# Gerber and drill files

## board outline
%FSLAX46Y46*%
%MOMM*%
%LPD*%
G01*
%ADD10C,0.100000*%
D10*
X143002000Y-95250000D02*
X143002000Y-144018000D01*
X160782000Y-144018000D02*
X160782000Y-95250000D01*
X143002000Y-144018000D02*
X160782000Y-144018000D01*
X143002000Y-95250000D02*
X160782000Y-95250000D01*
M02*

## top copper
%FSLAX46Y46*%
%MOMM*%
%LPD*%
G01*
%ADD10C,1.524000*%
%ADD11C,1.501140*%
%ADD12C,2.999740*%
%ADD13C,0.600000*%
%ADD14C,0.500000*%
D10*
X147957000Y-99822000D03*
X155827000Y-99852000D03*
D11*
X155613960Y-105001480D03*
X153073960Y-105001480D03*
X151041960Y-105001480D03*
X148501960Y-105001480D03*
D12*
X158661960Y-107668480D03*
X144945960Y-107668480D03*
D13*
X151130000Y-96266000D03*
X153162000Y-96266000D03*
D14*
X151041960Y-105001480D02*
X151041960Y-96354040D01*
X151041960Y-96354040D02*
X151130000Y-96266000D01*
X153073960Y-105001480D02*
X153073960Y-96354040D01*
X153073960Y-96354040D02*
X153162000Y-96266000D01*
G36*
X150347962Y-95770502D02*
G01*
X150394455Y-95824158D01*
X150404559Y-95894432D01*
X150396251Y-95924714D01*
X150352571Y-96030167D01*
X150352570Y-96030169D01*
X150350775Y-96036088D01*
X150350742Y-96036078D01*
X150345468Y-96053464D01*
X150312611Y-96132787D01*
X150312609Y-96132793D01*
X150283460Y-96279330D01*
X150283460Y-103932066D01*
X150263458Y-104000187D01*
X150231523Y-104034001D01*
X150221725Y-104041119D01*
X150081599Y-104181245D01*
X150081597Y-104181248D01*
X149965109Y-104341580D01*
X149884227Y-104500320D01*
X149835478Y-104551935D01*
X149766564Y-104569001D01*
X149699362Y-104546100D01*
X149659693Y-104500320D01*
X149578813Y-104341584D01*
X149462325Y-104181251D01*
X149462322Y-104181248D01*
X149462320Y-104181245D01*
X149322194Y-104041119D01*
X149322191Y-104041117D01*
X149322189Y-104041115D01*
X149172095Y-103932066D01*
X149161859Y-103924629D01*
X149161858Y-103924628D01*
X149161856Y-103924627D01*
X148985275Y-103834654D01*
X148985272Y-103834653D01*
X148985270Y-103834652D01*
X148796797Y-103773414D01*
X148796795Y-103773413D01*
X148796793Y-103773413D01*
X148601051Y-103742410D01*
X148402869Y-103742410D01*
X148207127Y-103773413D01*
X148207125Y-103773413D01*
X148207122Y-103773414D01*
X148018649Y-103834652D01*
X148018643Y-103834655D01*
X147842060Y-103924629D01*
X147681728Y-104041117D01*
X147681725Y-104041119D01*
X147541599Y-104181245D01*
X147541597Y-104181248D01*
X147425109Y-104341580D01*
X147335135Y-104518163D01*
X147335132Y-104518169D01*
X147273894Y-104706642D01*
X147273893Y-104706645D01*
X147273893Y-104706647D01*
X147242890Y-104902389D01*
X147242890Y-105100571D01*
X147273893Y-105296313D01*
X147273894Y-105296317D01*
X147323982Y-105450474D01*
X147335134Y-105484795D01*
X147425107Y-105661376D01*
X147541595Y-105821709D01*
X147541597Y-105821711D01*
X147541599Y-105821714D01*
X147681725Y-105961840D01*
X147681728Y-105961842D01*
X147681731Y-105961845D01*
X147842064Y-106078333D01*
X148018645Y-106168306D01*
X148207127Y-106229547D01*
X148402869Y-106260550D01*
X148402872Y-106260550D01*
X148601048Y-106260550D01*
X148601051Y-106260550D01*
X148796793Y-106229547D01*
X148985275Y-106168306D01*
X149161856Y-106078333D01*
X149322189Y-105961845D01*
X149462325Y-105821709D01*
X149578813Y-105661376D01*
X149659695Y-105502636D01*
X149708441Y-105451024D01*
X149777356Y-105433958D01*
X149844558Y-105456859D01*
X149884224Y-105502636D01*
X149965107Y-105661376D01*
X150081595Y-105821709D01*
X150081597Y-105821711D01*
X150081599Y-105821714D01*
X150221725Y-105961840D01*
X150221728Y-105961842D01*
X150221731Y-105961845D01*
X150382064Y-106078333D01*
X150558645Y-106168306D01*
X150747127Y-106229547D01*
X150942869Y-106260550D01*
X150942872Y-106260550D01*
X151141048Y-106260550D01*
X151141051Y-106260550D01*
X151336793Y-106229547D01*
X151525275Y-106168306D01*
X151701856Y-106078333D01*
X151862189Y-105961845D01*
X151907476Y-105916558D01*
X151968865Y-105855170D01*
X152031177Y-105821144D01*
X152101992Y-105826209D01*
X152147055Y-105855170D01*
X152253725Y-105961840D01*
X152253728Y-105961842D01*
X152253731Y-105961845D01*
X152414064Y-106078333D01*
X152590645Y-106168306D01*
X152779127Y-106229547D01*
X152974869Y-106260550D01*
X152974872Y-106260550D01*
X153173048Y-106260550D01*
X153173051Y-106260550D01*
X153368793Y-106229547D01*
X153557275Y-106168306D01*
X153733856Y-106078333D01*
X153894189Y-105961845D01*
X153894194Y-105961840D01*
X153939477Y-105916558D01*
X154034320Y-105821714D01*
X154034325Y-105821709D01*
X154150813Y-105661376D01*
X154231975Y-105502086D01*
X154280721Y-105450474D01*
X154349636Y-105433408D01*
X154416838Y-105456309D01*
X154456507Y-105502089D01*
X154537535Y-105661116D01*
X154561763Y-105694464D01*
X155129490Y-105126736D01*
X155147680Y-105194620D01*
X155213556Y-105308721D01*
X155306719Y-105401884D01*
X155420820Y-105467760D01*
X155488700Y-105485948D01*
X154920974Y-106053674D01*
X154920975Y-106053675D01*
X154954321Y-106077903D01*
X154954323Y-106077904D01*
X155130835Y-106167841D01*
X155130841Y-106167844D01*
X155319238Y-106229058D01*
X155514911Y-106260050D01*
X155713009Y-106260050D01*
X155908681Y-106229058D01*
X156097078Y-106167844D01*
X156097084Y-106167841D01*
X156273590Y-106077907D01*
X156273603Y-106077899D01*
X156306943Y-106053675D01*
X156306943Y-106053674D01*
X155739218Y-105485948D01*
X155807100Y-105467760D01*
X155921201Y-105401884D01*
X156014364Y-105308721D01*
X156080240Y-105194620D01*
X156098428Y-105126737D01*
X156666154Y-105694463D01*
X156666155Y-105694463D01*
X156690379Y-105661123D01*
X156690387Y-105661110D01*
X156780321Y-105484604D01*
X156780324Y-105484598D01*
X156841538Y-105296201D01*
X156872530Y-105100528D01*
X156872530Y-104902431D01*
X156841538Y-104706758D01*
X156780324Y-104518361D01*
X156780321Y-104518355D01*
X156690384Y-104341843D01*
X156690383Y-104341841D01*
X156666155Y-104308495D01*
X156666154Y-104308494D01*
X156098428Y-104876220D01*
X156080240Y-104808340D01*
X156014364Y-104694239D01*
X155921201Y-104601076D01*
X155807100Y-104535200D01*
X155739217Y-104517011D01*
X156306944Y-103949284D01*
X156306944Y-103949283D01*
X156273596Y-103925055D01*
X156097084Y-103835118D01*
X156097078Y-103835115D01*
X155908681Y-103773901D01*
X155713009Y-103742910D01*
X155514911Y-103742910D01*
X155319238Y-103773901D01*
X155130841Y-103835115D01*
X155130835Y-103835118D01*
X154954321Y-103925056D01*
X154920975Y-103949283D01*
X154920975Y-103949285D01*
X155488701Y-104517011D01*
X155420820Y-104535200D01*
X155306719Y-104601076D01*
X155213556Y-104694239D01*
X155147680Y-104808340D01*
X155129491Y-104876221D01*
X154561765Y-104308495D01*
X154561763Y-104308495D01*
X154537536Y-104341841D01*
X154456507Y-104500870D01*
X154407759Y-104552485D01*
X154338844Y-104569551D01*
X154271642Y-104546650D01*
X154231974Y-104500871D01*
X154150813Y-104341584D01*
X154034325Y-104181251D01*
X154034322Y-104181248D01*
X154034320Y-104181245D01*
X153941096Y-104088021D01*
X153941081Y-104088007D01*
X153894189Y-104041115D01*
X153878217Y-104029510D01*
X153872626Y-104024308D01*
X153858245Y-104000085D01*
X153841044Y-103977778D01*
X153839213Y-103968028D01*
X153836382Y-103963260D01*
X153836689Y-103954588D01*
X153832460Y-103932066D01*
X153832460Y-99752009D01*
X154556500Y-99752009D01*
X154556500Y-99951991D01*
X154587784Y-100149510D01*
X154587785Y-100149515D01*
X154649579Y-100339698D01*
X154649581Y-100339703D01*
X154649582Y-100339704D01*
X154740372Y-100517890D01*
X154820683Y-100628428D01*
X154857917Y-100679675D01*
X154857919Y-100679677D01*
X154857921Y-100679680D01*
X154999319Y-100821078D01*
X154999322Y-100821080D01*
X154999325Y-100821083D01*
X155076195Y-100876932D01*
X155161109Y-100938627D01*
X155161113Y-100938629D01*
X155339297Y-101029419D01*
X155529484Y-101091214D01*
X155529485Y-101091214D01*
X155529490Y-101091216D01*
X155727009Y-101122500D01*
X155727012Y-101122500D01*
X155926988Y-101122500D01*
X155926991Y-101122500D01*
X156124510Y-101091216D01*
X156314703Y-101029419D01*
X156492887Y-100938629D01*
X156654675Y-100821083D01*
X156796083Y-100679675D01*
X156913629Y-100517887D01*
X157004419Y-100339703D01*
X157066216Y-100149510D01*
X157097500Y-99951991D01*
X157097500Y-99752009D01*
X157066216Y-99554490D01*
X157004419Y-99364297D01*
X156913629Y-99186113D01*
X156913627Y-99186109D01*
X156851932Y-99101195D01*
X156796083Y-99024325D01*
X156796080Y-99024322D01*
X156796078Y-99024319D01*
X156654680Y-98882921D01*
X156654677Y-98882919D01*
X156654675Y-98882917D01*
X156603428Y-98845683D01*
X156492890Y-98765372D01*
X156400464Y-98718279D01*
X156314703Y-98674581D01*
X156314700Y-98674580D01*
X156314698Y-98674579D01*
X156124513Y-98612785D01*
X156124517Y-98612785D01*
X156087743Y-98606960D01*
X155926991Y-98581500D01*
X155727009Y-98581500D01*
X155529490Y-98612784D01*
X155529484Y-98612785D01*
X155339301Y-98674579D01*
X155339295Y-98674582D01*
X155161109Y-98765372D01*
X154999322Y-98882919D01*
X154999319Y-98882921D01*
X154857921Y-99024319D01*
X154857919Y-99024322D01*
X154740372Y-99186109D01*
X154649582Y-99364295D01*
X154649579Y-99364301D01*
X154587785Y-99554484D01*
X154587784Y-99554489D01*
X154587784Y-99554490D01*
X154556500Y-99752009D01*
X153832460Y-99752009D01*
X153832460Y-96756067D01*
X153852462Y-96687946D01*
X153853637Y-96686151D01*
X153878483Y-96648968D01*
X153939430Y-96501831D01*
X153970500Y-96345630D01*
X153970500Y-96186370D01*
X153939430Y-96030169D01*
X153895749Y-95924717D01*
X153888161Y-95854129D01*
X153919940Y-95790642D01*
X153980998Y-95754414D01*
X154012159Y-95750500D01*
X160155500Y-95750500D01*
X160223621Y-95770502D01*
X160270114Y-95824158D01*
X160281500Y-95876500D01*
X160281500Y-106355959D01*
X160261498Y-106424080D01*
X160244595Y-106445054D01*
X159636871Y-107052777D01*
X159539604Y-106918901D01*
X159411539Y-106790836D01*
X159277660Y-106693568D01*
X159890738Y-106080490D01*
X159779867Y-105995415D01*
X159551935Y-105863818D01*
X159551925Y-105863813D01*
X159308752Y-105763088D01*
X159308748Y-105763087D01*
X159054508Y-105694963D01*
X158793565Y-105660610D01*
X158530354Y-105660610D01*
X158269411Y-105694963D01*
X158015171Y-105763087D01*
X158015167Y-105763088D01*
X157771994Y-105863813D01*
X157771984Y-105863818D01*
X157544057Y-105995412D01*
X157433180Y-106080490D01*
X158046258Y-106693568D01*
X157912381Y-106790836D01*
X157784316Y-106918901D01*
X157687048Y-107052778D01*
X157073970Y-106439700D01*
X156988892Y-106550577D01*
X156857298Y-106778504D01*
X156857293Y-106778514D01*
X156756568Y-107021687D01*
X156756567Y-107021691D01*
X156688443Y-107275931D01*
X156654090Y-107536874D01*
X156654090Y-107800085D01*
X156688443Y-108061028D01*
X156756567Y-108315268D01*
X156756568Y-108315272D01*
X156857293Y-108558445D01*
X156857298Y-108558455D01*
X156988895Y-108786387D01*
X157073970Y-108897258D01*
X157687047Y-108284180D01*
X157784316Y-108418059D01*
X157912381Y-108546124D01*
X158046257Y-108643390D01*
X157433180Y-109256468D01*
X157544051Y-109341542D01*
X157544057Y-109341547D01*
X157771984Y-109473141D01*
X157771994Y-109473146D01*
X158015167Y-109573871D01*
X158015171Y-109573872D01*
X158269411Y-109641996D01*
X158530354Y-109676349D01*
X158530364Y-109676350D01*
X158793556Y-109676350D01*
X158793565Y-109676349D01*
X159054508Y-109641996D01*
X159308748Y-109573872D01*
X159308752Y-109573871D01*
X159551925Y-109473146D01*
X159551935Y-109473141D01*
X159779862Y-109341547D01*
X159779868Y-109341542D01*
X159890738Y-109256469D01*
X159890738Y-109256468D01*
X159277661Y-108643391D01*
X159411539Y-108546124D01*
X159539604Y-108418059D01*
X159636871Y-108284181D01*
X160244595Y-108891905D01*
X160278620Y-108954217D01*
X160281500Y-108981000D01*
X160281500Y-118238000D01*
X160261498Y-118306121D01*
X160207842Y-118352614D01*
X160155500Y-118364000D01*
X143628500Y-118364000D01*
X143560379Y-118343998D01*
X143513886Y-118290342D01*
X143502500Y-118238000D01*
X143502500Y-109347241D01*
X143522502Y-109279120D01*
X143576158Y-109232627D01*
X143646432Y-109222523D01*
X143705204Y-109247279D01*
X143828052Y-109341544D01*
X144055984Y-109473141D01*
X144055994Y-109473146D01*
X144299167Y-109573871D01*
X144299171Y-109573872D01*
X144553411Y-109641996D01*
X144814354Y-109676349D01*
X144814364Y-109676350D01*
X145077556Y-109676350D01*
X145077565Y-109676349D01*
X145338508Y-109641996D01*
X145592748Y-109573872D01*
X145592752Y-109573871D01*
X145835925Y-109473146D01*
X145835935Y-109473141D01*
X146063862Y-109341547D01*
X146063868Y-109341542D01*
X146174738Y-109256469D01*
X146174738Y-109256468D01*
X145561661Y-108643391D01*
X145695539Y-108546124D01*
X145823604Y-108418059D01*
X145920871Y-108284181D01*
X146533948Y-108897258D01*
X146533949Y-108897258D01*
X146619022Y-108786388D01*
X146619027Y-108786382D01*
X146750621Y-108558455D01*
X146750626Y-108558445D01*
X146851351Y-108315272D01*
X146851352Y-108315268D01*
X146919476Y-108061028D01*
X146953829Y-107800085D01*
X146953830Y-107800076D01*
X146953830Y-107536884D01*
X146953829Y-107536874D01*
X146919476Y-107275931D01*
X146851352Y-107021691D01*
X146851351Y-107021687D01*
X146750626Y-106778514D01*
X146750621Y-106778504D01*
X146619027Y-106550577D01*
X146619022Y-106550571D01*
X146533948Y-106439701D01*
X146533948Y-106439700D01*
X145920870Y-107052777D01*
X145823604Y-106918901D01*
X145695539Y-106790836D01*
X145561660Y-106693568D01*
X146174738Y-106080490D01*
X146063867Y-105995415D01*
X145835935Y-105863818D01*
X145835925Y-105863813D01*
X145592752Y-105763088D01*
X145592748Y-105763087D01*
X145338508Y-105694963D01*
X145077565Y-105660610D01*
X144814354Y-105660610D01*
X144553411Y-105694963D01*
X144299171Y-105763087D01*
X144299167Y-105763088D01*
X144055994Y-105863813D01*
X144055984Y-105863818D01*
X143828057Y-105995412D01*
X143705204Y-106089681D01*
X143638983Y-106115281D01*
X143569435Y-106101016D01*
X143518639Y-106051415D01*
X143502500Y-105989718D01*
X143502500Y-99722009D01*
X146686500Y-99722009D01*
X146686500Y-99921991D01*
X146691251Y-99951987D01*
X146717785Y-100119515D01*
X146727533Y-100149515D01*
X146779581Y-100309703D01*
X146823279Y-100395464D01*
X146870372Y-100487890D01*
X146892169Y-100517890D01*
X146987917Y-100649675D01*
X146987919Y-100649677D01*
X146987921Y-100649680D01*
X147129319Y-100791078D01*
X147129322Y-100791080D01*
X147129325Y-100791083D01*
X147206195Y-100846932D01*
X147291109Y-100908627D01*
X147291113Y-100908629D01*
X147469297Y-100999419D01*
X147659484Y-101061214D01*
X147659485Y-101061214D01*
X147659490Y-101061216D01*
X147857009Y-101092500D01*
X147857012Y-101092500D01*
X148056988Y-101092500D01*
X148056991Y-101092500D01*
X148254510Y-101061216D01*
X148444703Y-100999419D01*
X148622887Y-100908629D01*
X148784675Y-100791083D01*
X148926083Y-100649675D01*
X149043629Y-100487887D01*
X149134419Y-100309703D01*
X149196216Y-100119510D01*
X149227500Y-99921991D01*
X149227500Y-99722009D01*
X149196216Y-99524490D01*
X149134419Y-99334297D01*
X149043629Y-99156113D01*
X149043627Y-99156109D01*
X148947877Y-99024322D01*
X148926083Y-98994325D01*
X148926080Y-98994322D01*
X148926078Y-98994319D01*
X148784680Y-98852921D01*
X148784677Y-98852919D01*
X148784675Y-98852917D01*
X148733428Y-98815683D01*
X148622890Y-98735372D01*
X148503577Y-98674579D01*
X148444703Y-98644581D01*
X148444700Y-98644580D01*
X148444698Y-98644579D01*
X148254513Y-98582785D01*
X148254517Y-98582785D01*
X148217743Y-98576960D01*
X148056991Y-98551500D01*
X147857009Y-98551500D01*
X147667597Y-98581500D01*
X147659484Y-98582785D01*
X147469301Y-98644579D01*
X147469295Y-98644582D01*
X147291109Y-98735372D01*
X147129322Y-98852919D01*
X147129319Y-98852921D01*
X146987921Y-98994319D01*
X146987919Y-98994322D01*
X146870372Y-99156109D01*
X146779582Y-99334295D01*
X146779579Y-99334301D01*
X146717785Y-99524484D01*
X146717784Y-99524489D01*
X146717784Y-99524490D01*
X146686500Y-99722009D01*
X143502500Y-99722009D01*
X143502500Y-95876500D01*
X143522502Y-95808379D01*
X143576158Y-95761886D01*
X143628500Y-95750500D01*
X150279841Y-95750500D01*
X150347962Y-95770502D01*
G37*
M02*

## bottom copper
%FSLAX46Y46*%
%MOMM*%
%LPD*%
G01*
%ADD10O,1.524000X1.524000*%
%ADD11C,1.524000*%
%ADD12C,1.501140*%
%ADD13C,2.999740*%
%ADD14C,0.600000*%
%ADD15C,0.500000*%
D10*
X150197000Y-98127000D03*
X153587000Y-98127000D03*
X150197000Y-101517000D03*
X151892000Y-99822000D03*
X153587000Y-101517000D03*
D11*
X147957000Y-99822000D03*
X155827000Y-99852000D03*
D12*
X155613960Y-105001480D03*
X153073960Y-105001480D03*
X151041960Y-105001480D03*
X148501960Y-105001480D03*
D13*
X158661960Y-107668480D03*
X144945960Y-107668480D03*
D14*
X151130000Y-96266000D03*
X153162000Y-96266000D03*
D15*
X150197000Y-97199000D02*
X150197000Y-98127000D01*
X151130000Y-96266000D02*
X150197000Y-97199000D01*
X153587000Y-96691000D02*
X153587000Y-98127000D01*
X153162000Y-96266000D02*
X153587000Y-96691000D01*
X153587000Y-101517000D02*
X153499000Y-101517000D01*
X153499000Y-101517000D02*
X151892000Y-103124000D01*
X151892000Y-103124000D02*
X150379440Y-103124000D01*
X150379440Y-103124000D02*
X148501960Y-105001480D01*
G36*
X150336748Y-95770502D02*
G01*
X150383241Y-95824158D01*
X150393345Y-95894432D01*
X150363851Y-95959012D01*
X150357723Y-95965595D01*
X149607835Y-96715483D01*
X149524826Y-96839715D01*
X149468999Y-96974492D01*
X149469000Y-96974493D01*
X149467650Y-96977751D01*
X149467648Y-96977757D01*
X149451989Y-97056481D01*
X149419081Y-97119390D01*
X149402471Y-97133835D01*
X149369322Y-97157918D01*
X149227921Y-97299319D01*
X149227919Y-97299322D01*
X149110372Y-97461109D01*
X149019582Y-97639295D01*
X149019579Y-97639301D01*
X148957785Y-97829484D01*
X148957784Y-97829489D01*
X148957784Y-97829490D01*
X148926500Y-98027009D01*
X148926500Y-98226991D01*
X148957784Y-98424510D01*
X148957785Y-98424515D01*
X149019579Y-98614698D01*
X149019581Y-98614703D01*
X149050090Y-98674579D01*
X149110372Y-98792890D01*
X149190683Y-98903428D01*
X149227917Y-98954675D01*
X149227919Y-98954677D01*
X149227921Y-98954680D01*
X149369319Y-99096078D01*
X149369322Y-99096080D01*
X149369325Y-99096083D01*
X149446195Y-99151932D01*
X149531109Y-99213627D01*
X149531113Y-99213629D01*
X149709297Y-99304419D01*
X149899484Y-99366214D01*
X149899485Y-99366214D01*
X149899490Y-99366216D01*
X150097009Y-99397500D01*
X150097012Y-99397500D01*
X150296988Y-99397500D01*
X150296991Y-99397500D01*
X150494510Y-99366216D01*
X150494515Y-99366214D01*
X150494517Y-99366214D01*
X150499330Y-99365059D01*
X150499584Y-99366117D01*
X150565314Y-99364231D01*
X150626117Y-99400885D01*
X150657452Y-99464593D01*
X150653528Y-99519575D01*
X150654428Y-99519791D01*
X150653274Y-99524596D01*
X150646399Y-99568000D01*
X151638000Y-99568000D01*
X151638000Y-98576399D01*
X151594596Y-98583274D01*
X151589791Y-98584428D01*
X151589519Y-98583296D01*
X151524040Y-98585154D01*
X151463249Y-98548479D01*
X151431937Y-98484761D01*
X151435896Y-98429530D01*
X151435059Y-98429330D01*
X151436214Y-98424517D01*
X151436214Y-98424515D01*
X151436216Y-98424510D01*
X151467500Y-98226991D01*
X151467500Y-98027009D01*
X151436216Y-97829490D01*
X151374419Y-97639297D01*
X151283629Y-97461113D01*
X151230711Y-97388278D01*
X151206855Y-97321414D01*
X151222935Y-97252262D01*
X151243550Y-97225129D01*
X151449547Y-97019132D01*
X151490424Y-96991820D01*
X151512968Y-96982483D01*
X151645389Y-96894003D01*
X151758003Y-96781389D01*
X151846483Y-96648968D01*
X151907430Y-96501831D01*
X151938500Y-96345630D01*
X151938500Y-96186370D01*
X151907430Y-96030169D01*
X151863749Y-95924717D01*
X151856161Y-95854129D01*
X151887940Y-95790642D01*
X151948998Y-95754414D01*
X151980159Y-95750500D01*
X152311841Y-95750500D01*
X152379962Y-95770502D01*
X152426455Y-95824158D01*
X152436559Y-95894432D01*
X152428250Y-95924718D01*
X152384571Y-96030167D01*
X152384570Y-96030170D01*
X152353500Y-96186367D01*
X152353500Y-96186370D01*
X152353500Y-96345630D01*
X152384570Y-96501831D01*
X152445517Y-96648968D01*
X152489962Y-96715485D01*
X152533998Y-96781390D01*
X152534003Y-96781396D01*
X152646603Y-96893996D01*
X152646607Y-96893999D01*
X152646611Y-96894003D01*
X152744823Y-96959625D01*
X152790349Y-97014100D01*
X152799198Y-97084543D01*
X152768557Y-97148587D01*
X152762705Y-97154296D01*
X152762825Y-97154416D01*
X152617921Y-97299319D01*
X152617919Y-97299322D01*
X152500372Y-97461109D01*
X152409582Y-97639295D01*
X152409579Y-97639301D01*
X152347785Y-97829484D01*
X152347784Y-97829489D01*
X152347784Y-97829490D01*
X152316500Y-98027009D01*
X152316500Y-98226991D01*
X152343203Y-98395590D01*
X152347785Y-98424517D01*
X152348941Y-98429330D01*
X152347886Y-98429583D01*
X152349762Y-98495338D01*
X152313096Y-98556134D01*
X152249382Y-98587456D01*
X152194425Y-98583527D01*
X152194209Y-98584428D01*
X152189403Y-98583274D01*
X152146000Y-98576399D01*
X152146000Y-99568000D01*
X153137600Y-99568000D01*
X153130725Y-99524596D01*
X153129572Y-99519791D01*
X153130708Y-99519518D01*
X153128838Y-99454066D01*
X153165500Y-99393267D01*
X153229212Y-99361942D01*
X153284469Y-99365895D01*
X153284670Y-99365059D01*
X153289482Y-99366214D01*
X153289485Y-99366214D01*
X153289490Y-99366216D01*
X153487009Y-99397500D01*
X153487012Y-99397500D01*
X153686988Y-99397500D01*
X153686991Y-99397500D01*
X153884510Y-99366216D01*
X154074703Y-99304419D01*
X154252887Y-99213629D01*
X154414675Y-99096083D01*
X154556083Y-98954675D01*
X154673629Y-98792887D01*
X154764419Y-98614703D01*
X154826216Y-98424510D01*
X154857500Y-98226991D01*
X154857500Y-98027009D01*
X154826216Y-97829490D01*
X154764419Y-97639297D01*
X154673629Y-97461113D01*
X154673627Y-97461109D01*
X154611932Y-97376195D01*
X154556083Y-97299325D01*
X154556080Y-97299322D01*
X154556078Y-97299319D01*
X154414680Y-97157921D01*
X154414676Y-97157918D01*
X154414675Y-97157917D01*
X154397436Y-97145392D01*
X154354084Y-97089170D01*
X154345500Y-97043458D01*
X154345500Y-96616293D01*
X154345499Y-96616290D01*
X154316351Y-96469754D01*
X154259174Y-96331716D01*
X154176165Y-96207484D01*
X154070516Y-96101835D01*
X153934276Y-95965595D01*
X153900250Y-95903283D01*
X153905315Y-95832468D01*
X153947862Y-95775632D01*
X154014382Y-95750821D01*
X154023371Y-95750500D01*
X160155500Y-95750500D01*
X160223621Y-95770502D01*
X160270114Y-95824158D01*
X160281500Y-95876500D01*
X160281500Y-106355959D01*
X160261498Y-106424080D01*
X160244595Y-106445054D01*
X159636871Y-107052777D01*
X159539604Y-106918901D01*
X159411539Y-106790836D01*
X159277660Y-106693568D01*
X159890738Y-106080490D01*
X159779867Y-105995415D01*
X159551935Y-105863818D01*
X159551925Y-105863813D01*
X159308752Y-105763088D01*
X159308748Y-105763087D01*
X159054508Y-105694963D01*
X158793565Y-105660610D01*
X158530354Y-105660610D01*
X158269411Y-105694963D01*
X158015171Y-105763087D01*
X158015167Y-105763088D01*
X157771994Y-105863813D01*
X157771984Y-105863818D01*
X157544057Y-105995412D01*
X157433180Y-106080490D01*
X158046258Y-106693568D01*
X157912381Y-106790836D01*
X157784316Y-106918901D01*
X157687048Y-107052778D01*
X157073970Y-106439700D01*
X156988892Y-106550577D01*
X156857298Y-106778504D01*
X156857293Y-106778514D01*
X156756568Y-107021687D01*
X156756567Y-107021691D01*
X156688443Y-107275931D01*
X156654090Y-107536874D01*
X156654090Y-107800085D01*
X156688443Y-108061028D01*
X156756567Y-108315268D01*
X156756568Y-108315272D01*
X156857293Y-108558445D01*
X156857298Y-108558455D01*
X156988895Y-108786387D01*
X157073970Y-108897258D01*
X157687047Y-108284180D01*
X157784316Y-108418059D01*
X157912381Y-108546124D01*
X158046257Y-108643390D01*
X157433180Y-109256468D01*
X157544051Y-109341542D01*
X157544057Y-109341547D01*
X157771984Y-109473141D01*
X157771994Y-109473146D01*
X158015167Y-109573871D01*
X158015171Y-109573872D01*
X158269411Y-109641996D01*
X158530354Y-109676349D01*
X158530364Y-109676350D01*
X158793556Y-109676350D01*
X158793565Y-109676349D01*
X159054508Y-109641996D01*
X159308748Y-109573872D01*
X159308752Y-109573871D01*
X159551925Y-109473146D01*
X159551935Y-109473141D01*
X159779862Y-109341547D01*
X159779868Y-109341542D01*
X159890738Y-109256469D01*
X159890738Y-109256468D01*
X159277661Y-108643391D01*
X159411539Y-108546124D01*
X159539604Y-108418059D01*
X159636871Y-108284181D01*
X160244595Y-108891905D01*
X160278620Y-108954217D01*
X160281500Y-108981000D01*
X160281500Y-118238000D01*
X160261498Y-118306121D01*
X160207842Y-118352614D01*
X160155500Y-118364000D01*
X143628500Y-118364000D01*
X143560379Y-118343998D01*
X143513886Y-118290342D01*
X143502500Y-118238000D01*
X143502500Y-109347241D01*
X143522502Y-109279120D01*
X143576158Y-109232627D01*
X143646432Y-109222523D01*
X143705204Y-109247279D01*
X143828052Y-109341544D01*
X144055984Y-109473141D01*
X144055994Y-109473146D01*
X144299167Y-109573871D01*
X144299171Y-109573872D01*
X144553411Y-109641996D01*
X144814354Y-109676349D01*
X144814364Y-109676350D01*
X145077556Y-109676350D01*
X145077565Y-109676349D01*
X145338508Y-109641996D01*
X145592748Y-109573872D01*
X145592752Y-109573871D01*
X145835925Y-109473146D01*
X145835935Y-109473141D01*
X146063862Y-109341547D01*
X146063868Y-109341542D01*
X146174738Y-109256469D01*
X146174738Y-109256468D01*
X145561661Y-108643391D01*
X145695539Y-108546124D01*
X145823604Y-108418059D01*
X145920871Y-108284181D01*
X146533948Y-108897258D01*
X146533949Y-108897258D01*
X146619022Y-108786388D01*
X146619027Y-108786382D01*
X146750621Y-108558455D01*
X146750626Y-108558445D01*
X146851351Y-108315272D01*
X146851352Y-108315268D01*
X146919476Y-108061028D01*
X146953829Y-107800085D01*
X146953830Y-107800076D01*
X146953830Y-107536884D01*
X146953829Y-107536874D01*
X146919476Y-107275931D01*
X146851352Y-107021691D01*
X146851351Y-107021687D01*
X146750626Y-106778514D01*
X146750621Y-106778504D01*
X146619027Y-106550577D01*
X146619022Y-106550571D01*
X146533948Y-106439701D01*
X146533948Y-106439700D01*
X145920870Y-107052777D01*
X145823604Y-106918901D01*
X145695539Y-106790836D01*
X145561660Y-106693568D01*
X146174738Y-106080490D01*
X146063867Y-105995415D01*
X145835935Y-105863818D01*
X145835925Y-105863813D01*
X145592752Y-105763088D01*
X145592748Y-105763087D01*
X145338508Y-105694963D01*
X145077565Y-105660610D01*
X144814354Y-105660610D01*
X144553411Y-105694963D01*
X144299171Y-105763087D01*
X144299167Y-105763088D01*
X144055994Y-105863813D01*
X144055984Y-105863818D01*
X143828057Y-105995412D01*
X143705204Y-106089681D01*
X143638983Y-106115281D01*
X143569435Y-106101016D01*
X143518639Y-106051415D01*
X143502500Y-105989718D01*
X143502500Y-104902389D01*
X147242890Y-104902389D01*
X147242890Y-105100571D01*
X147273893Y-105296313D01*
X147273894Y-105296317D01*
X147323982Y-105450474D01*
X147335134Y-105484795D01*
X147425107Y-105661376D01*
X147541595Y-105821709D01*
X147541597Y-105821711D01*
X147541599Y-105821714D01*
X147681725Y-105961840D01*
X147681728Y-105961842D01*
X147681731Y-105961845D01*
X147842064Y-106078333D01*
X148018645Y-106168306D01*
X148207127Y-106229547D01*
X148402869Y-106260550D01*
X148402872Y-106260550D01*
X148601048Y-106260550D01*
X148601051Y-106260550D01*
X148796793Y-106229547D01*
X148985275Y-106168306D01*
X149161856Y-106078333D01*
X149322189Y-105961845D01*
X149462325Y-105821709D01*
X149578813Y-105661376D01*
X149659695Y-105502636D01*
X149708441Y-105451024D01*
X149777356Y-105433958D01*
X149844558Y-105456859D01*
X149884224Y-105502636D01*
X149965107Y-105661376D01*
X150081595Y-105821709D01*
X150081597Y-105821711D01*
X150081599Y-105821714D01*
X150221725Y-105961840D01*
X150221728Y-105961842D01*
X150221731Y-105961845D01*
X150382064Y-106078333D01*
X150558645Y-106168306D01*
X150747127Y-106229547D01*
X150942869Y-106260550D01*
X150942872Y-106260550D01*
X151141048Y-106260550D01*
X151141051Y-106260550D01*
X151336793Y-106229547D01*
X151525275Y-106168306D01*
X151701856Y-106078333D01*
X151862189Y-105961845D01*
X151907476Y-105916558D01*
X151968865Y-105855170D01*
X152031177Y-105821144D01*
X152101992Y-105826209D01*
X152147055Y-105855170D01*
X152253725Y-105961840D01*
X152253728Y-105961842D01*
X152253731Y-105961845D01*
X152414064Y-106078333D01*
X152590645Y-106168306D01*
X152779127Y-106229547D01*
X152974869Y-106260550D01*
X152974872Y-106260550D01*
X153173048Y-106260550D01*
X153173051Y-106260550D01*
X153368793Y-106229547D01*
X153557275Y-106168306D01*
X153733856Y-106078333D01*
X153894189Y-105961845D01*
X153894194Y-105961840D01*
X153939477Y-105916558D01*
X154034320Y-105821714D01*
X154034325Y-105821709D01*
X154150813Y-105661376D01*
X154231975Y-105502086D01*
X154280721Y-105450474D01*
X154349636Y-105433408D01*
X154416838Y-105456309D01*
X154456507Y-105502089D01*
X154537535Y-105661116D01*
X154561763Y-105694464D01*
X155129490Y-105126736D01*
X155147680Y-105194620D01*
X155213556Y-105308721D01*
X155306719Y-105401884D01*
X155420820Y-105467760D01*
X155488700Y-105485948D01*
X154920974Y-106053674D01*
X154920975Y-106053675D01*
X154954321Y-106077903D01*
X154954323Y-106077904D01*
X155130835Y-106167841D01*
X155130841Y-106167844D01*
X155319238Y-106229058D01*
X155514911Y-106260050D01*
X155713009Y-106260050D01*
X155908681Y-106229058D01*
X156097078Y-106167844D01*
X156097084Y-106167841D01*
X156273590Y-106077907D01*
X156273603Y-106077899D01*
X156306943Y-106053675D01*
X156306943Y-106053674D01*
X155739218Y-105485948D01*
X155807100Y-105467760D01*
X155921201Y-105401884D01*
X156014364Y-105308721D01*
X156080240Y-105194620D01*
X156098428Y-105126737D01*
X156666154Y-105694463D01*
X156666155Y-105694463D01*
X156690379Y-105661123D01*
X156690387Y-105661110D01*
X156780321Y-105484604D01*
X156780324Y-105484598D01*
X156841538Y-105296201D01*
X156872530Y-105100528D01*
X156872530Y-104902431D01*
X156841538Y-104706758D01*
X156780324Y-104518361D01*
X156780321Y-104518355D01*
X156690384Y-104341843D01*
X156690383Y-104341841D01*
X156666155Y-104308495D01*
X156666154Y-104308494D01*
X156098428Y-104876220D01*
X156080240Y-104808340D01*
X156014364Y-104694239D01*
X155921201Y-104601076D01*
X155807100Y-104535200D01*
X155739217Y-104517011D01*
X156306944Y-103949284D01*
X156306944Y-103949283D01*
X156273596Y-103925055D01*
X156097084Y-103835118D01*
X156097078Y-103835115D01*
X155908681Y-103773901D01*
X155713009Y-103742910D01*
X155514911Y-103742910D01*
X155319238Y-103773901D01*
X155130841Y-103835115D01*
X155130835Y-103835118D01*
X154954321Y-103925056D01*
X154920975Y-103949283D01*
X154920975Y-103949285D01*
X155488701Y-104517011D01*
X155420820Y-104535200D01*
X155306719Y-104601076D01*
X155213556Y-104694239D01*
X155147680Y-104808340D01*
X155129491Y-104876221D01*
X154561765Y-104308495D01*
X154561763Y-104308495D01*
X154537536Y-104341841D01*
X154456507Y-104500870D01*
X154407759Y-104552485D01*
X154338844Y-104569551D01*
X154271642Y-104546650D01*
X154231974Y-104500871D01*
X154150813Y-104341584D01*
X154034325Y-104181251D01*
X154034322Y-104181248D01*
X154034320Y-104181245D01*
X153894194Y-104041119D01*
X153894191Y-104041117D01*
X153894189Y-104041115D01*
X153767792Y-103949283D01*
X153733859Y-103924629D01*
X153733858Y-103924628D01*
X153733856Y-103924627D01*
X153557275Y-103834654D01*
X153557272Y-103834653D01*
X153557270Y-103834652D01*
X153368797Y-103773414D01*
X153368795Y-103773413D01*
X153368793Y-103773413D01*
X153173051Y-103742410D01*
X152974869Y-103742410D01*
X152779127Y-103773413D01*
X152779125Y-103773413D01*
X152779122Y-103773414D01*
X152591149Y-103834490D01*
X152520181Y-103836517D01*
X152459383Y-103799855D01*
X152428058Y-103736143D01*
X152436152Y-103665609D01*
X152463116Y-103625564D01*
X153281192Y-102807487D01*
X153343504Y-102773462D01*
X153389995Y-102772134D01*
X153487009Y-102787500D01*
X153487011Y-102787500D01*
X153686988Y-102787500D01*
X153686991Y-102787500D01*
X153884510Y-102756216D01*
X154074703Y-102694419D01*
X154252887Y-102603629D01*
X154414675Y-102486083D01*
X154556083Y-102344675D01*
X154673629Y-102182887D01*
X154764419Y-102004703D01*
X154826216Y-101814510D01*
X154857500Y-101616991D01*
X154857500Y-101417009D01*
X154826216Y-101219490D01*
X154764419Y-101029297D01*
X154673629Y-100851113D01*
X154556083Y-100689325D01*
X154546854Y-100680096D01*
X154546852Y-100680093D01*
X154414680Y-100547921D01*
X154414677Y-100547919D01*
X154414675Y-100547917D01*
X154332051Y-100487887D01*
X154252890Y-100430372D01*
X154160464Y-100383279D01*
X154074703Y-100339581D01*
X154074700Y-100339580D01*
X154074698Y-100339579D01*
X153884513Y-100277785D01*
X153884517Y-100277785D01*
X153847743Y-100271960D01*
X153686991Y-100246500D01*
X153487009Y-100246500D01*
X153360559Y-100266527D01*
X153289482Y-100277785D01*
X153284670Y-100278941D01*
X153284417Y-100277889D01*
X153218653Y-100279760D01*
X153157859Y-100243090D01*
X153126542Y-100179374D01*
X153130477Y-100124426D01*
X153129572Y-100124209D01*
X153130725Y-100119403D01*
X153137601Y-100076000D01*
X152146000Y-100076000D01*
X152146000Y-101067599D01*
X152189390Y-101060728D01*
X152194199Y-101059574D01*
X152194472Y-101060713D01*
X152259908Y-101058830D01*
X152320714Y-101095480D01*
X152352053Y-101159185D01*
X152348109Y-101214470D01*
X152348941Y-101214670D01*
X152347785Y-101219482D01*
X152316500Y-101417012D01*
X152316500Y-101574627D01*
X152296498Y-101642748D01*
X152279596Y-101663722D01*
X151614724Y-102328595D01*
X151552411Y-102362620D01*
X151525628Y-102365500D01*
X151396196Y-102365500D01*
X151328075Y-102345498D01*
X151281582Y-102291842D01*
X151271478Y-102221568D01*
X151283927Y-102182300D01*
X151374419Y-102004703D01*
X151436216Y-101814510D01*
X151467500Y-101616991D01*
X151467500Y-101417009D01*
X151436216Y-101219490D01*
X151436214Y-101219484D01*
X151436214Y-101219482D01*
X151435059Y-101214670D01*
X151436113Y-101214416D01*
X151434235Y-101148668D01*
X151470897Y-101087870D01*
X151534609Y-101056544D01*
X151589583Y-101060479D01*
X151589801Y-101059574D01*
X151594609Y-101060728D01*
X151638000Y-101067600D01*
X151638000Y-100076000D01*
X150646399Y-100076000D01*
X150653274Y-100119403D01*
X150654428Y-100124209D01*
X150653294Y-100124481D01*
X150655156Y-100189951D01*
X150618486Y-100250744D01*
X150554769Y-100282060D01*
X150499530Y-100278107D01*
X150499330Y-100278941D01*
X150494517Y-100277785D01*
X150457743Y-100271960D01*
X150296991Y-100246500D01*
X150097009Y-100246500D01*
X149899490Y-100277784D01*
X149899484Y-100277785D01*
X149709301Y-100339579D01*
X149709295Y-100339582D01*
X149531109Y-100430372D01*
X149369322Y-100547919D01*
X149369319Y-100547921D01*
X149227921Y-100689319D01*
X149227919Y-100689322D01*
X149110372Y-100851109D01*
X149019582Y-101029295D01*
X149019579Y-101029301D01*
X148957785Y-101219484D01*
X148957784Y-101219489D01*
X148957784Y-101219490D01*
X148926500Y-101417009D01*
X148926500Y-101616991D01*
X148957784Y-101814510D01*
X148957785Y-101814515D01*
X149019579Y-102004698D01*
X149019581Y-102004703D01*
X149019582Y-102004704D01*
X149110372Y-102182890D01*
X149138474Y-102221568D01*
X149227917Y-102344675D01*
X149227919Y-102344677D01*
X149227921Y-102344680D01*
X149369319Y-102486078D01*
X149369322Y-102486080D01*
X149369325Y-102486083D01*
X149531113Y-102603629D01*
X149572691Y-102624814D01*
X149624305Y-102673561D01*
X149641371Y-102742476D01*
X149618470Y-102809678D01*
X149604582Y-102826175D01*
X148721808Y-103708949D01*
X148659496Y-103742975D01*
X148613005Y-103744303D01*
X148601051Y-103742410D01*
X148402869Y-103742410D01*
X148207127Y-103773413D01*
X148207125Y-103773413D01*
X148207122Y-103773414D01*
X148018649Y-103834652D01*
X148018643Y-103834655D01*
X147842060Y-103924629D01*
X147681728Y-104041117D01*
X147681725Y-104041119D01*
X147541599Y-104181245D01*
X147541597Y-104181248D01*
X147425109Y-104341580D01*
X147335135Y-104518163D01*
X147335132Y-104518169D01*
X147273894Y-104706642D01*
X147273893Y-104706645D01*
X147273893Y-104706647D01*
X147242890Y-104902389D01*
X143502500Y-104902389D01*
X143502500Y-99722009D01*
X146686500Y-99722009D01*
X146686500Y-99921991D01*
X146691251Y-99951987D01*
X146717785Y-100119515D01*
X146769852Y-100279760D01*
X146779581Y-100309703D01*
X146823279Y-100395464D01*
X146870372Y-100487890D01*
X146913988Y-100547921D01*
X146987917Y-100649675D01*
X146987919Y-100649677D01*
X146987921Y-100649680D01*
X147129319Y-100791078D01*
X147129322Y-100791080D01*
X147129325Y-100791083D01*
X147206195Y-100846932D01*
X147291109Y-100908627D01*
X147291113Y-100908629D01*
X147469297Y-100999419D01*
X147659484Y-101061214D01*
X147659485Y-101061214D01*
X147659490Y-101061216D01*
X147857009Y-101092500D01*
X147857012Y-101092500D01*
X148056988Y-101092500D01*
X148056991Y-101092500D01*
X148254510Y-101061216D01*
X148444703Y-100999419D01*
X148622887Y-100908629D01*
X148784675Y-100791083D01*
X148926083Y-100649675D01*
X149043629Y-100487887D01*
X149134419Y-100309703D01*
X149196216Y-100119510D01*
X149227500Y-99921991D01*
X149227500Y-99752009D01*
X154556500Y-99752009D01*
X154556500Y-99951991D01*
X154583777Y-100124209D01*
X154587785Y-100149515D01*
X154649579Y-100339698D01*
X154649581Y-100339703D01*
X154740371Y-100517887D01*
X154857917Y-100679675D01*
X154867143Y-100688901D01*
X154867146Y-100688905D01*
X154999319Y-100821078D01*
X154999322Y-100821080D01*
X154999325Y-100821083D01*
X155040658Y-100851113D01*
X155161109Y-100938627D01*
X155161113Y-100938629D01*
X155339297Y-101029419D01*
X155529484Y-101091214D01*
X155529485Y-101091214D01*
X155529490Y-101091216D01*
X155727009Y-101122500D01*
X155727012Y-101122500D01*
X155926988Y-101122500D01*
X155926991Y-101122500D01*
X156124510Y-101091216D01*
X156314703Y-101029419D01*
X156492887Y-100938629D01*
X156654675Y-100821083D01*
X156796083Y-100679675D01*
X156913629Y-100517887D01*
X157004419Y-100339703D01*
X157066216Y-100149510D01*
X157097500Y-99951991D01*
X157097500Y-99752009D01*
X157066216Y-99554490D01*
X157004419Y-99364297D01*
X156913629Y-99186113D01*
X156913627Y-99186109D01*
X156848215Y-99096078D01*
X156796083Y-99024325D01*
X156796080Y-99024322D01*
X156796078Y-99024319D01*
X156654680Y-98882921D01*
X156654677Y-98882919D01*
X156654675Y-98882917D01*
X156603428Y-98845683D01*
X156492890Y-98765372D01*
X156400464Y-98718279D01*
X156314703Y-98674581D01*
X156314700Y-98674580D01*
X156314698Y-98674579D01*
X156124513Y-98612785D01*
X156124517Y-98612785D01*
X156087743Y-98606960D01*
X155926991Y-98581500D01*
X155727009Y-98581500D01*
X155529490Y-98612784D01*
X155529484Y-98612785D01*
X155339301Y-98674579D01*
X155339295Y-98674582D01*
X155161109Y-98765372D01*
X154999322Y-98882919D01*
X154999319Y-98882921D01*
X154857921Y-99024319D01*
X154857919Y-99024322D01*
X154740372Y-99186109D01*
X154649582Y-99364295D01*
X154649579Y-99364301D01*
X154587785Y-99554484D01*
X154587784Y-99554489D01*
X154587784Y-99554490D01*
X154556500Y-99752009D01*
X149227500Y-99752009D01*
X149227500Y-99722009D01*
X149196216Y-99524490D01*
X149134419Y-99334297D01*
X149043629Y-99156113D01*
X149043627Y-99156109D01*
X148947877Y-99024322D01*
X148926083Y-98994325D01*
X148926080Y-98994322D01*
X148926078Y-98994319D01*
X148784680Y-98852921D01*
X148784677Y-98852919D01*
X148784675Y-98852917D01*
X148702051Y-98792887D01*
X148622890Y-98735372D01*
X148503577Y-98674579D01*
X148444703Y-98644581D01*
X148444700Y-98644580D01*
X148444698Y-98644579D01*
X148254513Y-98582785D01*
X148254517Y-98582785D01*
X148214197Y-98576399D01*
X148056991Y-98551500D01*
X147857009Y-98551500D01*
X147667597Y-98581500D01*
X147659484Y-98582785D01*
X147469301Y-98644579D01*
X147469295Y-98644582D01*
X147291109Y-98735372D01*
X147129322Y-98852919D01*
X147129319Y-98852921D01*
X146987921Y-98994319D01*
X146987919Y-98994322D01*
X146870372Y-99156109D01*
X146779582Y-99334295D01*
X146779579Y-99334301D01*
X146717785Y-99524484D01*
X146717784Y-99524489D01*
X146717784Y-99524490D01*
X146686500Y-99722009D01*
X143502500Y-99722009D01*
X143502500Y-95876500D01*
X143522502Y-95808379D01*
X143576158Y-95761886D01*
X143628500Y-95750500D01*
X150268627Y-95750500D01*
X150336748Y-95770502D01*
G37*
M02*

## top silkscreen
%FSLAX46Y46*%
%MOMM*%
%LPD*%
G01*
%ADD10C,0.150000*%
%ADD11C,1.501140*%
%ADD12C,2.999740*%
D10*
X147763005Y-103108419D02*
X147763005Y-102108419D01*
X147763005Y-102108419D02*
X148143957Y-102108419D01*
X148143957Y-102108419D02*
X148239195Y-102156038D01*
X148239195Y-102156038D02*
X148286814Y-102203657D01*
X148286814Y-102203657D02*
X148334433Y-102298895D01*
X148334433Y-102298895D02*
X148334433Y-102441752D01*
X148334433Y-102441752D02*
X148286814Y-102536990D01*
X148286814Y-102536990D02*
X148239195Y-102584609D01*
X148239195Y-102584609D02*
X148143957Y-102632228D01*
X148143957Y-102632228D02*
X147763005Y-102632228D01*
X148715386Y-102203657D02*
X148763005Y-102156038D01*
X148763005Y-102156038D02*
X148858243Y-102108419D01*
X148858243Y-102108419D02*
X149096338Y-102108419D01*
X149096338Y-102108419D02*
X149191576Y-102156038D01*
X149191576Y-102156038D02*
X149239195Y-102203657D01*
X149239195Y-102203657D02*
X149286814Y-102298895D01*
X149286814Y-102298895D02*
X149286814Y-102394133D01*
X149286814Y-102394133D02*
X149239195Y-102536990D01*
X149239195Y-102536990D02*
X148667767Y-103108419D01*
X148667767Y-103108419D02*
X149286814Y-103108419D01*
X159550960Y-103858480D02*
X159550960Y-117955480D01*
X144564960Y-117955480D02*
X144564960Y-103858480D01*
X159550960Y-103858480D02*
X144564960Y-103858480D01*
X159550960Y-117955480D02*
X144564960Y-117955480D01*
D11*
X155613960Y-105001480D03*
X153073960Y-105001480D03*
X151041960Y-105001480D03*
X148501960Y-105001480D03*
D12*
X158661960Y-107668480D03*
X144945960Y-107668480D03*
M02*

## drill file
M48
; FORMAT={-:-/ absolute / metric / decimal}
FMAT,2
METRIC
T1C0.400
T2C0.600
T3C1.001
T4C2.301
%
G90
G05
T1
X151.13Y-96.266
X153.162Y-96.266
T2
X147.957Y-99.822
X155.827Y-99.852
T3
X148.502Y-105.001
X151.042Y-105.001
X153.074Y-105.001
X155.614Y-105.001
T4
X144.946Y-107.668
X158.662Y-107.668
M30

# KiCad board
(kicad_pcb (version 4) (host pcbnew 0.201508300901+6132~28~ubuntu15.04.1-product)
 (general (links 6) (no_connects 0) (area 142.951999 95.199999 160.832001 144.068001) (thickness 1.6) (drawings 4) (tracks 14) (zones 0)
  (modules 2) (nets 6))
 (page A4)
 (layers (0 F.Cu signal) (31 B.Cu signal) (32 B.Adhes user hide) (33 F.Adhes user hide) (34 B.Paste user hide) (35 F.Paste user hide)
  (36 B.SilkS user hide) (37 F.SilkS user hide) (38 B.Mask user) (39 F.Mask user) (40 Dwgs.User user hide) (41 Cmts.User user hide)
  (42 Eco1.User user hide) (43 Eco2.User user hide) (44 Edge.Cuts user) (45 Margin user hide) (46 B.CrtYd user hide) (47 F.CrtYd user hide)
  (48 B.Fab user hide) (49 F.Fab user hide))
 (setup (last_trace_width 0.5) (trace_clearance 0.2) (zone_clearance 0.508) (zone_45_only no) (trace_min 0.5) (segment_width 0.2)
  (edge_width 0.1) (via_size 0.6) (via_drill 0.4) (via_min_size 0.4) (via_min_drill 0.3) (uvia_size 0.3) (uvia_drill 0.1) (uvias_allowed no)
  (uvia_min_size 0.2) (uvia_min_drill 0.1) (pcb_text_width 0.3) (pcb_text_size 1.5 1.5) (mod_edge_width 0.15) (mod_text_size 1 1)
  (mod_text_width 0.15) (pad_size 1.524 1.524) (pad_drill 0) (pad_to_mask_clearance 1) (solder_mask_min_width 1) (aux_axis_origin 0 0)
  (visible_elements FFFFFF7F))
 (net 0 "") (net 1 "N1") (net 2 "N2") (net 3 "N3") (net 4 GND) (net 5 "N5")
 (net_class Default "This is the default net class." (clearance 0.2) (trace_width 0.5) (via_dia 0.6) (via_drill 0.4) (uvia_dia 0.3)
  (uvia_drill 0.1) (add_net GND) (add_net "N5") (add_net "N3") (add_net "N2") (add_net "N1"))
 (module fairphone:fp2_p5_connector (layer B.Cu) (at 151.892 99.822)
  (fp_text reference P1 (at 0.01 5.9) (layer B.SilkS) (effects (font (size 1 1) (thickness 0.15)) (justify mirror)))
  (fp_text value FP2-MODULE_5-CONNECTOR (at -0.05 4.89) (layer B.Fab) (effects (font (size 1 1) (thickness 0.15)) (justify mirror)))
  (pad 5 smd oval (at -1.695 -1.695) (size 1.524 1.524) (layers B.Cu B.Paste B.Mask) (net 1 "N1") (solder_mask_margin 1))
  (pad 4 smd oval (at 1.695 -1.695) (size 1.524 1.524) (layers B.Cu B.Paste) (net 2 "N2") (solder_mask_margin 1))
  (pad 2 smd oval (at -1.695 1.695) (size 1.524 1.524) (layers B.Cu B.Paste B.Mask) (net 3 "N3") (solder_mask_margin 1))
  (pad 3 smd oval (at 0 0) (size 1.524 1.524) (layers B.Cu B.Paste B.Mask) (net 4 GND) (solder_mask_margin 1))
  (pad 1 smd oval (at 1.695 1.695) (size 1.524 1.524) (layers B.Cu B.Paste B.Mask) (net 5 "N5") (solder_mask_margin 1))
  (pad "" thru_hole circle (at -3.935 0) (size 1.524 1.524) (drill 0.6) (layers *.Cu *.Mask B.SilkS))
  (pad "" thru_hole circle (at 3.935 0.03) (size 1.524 1.524) (drill 0.6) (layers *.Cu *.Mask B.SilkS)))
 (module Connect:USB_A (layer F.Cu) (at 148.5011 105.0036)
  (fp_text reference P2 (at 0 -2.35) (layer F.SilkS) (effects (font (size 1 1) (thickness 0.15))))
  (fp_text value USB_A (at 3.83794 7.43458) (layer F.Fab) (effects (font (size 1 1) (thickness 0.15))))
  (fp_line (start 11.04986 -1.14512) (end 11.04986 12.95188) (layer F.SilkS) (width 0.15))
  (fp_line (start -3.93614 12.95188) (end -3.93614 -1.14512) (layer F.SilkS) (width 0.15))
  (fp_line (start 11.04986 -1.14512) (end -3.93614 -1.14512) (layer F.SilkS) (width 0.15))
  (fp_line (start 11.04986 12.95188) (end -3.93614 12.95188) (layer F.SilkS) (width 0.15))
  (pad 4 thru_hole circle (at 7.11286 -0.00212 270) (size 1.50114 1.50114) (drill 1.00076) (layers *.Cu *.Mask F.SilkS) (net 4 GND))
  (pad 3 thru_hole circle (at 4.57286 -0.00212 270) (size 1.50114 1.50114) (drill 1.00076) (layers *.Cu *.Mask F.SilkS) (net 2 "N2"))
  (pad 2 thru_hole circle (at 2.54086 -0.00212 270) (size 1.50114 1.50114) (drill 1.00076) (layers *.Cu *.Mask F.SilkS) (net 1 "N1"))
  (pad 1 thru_hole circle (at 0.00086 -0.00212 270) (size 1.50114 1.50114) (drill 1.00076) (layers *.Cu *.Mask F.SilkS) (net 5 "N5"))
  (pad 5 thru_hole circle (at 10.16086 2.66488 270) (size 2.99974 2.99974) (drill 2.30124) (layers *.Cu *.Mask F.SilkS) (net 4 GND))
  (pad 5 thru_hole circle (at -3.55514 2.66488 270) (size 2.99974 2.99974) (drill 2.30124) (layers *.Cu *.Mask F.SilkS) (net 4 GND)))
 (gr_line (start 143.002 95.25) (end 143.002 144.018) (angle 90) (layer Edge.Cuts) (width 0.1))
 (gr_line (start 160.782 144.018) (end 160.782 95.25) (angle 90) (layer Edge.Cuts) (width 0.1))
 (gr_line (start 143.002 144.018) (end 160.782 144.018) (angle 90) (layer Edge.Cuts) (width 0.1))
 (gr_line (start 143.002 95.25) (end 160.782 95.25) (angle 90) (layer Edge.Cuts) (width 0.1))
 (segment (start 151.04196 105.00148) (end 151.04196 96.35404) (width 0.5) (layer F.Cu) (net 1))
 (segment (start 151.04196 96.35404) (end 151.13 96.266) (width 0.5) (layer F.Cu) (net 1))
 (segment (start 150.197 97.199) (end 150.197 98.127) (width 0.5) (layer B.Cu) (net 1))
 (segment (start 151.13 96.266) (end 150.197 97.199) (width 0.5) (layer B.Cu) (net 1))
 (via (at 151.13 96.266) (size 0.6) (drill 0.4) (layers F.Cu B.Cu) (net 1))
 (segment (start 153.07396 105.00148) (end 153.07396 96.35404) (width 0.5) (layer F.Cu) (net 2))
 (segment (start 153.587 96.691) (end 153.587 98.127) (width 0.5) (layer B.Cu) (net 2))
 (segment (start 153.162 96.266) (end 153.587 96.691) (width 0.5) (layer B.Cu) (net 2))
 (via (at 153.162 96.266) (size 0.6) (drill 0.4) (layers F.Cu B.Cu) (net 2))
 (segment (start 153.07396 96.35404) (end 153.162 96.266) (width 0.5) (layer F.Cu) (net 2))
 (segment (start 153.587 101.517) (end 153.499 101.517) (width 0.5) (layer B.Cu) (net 5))
 (segment (start 153.499 101.517) (end 151.892 103.124) (width 0.5) (layer B.Cu) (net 5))
 (segment (start 151.892 103.124) (end 150.37944 103.124) (width 0.5) (layer B.Cu) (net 5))
 (segment (start 150.37944 103.124) (end 148.50196 105.00148) (width 0.5) (layer B.Cu) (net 5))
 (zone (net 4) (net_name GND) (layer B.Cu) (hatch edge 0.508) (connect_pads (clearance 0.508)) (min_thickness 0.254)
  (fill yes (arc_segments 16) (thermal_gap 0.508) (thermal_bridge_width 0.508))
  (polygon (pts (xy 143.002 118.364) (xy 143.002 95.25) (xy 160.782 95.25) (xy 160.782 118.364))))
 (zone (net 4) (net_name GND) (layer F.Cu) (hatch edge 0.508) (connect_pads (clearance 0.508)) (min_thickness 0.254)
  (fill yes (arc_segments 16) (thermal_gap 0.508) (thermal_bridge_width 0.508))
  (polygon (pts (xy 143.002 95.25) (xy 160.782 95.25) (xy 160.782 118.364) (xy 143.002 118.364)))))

